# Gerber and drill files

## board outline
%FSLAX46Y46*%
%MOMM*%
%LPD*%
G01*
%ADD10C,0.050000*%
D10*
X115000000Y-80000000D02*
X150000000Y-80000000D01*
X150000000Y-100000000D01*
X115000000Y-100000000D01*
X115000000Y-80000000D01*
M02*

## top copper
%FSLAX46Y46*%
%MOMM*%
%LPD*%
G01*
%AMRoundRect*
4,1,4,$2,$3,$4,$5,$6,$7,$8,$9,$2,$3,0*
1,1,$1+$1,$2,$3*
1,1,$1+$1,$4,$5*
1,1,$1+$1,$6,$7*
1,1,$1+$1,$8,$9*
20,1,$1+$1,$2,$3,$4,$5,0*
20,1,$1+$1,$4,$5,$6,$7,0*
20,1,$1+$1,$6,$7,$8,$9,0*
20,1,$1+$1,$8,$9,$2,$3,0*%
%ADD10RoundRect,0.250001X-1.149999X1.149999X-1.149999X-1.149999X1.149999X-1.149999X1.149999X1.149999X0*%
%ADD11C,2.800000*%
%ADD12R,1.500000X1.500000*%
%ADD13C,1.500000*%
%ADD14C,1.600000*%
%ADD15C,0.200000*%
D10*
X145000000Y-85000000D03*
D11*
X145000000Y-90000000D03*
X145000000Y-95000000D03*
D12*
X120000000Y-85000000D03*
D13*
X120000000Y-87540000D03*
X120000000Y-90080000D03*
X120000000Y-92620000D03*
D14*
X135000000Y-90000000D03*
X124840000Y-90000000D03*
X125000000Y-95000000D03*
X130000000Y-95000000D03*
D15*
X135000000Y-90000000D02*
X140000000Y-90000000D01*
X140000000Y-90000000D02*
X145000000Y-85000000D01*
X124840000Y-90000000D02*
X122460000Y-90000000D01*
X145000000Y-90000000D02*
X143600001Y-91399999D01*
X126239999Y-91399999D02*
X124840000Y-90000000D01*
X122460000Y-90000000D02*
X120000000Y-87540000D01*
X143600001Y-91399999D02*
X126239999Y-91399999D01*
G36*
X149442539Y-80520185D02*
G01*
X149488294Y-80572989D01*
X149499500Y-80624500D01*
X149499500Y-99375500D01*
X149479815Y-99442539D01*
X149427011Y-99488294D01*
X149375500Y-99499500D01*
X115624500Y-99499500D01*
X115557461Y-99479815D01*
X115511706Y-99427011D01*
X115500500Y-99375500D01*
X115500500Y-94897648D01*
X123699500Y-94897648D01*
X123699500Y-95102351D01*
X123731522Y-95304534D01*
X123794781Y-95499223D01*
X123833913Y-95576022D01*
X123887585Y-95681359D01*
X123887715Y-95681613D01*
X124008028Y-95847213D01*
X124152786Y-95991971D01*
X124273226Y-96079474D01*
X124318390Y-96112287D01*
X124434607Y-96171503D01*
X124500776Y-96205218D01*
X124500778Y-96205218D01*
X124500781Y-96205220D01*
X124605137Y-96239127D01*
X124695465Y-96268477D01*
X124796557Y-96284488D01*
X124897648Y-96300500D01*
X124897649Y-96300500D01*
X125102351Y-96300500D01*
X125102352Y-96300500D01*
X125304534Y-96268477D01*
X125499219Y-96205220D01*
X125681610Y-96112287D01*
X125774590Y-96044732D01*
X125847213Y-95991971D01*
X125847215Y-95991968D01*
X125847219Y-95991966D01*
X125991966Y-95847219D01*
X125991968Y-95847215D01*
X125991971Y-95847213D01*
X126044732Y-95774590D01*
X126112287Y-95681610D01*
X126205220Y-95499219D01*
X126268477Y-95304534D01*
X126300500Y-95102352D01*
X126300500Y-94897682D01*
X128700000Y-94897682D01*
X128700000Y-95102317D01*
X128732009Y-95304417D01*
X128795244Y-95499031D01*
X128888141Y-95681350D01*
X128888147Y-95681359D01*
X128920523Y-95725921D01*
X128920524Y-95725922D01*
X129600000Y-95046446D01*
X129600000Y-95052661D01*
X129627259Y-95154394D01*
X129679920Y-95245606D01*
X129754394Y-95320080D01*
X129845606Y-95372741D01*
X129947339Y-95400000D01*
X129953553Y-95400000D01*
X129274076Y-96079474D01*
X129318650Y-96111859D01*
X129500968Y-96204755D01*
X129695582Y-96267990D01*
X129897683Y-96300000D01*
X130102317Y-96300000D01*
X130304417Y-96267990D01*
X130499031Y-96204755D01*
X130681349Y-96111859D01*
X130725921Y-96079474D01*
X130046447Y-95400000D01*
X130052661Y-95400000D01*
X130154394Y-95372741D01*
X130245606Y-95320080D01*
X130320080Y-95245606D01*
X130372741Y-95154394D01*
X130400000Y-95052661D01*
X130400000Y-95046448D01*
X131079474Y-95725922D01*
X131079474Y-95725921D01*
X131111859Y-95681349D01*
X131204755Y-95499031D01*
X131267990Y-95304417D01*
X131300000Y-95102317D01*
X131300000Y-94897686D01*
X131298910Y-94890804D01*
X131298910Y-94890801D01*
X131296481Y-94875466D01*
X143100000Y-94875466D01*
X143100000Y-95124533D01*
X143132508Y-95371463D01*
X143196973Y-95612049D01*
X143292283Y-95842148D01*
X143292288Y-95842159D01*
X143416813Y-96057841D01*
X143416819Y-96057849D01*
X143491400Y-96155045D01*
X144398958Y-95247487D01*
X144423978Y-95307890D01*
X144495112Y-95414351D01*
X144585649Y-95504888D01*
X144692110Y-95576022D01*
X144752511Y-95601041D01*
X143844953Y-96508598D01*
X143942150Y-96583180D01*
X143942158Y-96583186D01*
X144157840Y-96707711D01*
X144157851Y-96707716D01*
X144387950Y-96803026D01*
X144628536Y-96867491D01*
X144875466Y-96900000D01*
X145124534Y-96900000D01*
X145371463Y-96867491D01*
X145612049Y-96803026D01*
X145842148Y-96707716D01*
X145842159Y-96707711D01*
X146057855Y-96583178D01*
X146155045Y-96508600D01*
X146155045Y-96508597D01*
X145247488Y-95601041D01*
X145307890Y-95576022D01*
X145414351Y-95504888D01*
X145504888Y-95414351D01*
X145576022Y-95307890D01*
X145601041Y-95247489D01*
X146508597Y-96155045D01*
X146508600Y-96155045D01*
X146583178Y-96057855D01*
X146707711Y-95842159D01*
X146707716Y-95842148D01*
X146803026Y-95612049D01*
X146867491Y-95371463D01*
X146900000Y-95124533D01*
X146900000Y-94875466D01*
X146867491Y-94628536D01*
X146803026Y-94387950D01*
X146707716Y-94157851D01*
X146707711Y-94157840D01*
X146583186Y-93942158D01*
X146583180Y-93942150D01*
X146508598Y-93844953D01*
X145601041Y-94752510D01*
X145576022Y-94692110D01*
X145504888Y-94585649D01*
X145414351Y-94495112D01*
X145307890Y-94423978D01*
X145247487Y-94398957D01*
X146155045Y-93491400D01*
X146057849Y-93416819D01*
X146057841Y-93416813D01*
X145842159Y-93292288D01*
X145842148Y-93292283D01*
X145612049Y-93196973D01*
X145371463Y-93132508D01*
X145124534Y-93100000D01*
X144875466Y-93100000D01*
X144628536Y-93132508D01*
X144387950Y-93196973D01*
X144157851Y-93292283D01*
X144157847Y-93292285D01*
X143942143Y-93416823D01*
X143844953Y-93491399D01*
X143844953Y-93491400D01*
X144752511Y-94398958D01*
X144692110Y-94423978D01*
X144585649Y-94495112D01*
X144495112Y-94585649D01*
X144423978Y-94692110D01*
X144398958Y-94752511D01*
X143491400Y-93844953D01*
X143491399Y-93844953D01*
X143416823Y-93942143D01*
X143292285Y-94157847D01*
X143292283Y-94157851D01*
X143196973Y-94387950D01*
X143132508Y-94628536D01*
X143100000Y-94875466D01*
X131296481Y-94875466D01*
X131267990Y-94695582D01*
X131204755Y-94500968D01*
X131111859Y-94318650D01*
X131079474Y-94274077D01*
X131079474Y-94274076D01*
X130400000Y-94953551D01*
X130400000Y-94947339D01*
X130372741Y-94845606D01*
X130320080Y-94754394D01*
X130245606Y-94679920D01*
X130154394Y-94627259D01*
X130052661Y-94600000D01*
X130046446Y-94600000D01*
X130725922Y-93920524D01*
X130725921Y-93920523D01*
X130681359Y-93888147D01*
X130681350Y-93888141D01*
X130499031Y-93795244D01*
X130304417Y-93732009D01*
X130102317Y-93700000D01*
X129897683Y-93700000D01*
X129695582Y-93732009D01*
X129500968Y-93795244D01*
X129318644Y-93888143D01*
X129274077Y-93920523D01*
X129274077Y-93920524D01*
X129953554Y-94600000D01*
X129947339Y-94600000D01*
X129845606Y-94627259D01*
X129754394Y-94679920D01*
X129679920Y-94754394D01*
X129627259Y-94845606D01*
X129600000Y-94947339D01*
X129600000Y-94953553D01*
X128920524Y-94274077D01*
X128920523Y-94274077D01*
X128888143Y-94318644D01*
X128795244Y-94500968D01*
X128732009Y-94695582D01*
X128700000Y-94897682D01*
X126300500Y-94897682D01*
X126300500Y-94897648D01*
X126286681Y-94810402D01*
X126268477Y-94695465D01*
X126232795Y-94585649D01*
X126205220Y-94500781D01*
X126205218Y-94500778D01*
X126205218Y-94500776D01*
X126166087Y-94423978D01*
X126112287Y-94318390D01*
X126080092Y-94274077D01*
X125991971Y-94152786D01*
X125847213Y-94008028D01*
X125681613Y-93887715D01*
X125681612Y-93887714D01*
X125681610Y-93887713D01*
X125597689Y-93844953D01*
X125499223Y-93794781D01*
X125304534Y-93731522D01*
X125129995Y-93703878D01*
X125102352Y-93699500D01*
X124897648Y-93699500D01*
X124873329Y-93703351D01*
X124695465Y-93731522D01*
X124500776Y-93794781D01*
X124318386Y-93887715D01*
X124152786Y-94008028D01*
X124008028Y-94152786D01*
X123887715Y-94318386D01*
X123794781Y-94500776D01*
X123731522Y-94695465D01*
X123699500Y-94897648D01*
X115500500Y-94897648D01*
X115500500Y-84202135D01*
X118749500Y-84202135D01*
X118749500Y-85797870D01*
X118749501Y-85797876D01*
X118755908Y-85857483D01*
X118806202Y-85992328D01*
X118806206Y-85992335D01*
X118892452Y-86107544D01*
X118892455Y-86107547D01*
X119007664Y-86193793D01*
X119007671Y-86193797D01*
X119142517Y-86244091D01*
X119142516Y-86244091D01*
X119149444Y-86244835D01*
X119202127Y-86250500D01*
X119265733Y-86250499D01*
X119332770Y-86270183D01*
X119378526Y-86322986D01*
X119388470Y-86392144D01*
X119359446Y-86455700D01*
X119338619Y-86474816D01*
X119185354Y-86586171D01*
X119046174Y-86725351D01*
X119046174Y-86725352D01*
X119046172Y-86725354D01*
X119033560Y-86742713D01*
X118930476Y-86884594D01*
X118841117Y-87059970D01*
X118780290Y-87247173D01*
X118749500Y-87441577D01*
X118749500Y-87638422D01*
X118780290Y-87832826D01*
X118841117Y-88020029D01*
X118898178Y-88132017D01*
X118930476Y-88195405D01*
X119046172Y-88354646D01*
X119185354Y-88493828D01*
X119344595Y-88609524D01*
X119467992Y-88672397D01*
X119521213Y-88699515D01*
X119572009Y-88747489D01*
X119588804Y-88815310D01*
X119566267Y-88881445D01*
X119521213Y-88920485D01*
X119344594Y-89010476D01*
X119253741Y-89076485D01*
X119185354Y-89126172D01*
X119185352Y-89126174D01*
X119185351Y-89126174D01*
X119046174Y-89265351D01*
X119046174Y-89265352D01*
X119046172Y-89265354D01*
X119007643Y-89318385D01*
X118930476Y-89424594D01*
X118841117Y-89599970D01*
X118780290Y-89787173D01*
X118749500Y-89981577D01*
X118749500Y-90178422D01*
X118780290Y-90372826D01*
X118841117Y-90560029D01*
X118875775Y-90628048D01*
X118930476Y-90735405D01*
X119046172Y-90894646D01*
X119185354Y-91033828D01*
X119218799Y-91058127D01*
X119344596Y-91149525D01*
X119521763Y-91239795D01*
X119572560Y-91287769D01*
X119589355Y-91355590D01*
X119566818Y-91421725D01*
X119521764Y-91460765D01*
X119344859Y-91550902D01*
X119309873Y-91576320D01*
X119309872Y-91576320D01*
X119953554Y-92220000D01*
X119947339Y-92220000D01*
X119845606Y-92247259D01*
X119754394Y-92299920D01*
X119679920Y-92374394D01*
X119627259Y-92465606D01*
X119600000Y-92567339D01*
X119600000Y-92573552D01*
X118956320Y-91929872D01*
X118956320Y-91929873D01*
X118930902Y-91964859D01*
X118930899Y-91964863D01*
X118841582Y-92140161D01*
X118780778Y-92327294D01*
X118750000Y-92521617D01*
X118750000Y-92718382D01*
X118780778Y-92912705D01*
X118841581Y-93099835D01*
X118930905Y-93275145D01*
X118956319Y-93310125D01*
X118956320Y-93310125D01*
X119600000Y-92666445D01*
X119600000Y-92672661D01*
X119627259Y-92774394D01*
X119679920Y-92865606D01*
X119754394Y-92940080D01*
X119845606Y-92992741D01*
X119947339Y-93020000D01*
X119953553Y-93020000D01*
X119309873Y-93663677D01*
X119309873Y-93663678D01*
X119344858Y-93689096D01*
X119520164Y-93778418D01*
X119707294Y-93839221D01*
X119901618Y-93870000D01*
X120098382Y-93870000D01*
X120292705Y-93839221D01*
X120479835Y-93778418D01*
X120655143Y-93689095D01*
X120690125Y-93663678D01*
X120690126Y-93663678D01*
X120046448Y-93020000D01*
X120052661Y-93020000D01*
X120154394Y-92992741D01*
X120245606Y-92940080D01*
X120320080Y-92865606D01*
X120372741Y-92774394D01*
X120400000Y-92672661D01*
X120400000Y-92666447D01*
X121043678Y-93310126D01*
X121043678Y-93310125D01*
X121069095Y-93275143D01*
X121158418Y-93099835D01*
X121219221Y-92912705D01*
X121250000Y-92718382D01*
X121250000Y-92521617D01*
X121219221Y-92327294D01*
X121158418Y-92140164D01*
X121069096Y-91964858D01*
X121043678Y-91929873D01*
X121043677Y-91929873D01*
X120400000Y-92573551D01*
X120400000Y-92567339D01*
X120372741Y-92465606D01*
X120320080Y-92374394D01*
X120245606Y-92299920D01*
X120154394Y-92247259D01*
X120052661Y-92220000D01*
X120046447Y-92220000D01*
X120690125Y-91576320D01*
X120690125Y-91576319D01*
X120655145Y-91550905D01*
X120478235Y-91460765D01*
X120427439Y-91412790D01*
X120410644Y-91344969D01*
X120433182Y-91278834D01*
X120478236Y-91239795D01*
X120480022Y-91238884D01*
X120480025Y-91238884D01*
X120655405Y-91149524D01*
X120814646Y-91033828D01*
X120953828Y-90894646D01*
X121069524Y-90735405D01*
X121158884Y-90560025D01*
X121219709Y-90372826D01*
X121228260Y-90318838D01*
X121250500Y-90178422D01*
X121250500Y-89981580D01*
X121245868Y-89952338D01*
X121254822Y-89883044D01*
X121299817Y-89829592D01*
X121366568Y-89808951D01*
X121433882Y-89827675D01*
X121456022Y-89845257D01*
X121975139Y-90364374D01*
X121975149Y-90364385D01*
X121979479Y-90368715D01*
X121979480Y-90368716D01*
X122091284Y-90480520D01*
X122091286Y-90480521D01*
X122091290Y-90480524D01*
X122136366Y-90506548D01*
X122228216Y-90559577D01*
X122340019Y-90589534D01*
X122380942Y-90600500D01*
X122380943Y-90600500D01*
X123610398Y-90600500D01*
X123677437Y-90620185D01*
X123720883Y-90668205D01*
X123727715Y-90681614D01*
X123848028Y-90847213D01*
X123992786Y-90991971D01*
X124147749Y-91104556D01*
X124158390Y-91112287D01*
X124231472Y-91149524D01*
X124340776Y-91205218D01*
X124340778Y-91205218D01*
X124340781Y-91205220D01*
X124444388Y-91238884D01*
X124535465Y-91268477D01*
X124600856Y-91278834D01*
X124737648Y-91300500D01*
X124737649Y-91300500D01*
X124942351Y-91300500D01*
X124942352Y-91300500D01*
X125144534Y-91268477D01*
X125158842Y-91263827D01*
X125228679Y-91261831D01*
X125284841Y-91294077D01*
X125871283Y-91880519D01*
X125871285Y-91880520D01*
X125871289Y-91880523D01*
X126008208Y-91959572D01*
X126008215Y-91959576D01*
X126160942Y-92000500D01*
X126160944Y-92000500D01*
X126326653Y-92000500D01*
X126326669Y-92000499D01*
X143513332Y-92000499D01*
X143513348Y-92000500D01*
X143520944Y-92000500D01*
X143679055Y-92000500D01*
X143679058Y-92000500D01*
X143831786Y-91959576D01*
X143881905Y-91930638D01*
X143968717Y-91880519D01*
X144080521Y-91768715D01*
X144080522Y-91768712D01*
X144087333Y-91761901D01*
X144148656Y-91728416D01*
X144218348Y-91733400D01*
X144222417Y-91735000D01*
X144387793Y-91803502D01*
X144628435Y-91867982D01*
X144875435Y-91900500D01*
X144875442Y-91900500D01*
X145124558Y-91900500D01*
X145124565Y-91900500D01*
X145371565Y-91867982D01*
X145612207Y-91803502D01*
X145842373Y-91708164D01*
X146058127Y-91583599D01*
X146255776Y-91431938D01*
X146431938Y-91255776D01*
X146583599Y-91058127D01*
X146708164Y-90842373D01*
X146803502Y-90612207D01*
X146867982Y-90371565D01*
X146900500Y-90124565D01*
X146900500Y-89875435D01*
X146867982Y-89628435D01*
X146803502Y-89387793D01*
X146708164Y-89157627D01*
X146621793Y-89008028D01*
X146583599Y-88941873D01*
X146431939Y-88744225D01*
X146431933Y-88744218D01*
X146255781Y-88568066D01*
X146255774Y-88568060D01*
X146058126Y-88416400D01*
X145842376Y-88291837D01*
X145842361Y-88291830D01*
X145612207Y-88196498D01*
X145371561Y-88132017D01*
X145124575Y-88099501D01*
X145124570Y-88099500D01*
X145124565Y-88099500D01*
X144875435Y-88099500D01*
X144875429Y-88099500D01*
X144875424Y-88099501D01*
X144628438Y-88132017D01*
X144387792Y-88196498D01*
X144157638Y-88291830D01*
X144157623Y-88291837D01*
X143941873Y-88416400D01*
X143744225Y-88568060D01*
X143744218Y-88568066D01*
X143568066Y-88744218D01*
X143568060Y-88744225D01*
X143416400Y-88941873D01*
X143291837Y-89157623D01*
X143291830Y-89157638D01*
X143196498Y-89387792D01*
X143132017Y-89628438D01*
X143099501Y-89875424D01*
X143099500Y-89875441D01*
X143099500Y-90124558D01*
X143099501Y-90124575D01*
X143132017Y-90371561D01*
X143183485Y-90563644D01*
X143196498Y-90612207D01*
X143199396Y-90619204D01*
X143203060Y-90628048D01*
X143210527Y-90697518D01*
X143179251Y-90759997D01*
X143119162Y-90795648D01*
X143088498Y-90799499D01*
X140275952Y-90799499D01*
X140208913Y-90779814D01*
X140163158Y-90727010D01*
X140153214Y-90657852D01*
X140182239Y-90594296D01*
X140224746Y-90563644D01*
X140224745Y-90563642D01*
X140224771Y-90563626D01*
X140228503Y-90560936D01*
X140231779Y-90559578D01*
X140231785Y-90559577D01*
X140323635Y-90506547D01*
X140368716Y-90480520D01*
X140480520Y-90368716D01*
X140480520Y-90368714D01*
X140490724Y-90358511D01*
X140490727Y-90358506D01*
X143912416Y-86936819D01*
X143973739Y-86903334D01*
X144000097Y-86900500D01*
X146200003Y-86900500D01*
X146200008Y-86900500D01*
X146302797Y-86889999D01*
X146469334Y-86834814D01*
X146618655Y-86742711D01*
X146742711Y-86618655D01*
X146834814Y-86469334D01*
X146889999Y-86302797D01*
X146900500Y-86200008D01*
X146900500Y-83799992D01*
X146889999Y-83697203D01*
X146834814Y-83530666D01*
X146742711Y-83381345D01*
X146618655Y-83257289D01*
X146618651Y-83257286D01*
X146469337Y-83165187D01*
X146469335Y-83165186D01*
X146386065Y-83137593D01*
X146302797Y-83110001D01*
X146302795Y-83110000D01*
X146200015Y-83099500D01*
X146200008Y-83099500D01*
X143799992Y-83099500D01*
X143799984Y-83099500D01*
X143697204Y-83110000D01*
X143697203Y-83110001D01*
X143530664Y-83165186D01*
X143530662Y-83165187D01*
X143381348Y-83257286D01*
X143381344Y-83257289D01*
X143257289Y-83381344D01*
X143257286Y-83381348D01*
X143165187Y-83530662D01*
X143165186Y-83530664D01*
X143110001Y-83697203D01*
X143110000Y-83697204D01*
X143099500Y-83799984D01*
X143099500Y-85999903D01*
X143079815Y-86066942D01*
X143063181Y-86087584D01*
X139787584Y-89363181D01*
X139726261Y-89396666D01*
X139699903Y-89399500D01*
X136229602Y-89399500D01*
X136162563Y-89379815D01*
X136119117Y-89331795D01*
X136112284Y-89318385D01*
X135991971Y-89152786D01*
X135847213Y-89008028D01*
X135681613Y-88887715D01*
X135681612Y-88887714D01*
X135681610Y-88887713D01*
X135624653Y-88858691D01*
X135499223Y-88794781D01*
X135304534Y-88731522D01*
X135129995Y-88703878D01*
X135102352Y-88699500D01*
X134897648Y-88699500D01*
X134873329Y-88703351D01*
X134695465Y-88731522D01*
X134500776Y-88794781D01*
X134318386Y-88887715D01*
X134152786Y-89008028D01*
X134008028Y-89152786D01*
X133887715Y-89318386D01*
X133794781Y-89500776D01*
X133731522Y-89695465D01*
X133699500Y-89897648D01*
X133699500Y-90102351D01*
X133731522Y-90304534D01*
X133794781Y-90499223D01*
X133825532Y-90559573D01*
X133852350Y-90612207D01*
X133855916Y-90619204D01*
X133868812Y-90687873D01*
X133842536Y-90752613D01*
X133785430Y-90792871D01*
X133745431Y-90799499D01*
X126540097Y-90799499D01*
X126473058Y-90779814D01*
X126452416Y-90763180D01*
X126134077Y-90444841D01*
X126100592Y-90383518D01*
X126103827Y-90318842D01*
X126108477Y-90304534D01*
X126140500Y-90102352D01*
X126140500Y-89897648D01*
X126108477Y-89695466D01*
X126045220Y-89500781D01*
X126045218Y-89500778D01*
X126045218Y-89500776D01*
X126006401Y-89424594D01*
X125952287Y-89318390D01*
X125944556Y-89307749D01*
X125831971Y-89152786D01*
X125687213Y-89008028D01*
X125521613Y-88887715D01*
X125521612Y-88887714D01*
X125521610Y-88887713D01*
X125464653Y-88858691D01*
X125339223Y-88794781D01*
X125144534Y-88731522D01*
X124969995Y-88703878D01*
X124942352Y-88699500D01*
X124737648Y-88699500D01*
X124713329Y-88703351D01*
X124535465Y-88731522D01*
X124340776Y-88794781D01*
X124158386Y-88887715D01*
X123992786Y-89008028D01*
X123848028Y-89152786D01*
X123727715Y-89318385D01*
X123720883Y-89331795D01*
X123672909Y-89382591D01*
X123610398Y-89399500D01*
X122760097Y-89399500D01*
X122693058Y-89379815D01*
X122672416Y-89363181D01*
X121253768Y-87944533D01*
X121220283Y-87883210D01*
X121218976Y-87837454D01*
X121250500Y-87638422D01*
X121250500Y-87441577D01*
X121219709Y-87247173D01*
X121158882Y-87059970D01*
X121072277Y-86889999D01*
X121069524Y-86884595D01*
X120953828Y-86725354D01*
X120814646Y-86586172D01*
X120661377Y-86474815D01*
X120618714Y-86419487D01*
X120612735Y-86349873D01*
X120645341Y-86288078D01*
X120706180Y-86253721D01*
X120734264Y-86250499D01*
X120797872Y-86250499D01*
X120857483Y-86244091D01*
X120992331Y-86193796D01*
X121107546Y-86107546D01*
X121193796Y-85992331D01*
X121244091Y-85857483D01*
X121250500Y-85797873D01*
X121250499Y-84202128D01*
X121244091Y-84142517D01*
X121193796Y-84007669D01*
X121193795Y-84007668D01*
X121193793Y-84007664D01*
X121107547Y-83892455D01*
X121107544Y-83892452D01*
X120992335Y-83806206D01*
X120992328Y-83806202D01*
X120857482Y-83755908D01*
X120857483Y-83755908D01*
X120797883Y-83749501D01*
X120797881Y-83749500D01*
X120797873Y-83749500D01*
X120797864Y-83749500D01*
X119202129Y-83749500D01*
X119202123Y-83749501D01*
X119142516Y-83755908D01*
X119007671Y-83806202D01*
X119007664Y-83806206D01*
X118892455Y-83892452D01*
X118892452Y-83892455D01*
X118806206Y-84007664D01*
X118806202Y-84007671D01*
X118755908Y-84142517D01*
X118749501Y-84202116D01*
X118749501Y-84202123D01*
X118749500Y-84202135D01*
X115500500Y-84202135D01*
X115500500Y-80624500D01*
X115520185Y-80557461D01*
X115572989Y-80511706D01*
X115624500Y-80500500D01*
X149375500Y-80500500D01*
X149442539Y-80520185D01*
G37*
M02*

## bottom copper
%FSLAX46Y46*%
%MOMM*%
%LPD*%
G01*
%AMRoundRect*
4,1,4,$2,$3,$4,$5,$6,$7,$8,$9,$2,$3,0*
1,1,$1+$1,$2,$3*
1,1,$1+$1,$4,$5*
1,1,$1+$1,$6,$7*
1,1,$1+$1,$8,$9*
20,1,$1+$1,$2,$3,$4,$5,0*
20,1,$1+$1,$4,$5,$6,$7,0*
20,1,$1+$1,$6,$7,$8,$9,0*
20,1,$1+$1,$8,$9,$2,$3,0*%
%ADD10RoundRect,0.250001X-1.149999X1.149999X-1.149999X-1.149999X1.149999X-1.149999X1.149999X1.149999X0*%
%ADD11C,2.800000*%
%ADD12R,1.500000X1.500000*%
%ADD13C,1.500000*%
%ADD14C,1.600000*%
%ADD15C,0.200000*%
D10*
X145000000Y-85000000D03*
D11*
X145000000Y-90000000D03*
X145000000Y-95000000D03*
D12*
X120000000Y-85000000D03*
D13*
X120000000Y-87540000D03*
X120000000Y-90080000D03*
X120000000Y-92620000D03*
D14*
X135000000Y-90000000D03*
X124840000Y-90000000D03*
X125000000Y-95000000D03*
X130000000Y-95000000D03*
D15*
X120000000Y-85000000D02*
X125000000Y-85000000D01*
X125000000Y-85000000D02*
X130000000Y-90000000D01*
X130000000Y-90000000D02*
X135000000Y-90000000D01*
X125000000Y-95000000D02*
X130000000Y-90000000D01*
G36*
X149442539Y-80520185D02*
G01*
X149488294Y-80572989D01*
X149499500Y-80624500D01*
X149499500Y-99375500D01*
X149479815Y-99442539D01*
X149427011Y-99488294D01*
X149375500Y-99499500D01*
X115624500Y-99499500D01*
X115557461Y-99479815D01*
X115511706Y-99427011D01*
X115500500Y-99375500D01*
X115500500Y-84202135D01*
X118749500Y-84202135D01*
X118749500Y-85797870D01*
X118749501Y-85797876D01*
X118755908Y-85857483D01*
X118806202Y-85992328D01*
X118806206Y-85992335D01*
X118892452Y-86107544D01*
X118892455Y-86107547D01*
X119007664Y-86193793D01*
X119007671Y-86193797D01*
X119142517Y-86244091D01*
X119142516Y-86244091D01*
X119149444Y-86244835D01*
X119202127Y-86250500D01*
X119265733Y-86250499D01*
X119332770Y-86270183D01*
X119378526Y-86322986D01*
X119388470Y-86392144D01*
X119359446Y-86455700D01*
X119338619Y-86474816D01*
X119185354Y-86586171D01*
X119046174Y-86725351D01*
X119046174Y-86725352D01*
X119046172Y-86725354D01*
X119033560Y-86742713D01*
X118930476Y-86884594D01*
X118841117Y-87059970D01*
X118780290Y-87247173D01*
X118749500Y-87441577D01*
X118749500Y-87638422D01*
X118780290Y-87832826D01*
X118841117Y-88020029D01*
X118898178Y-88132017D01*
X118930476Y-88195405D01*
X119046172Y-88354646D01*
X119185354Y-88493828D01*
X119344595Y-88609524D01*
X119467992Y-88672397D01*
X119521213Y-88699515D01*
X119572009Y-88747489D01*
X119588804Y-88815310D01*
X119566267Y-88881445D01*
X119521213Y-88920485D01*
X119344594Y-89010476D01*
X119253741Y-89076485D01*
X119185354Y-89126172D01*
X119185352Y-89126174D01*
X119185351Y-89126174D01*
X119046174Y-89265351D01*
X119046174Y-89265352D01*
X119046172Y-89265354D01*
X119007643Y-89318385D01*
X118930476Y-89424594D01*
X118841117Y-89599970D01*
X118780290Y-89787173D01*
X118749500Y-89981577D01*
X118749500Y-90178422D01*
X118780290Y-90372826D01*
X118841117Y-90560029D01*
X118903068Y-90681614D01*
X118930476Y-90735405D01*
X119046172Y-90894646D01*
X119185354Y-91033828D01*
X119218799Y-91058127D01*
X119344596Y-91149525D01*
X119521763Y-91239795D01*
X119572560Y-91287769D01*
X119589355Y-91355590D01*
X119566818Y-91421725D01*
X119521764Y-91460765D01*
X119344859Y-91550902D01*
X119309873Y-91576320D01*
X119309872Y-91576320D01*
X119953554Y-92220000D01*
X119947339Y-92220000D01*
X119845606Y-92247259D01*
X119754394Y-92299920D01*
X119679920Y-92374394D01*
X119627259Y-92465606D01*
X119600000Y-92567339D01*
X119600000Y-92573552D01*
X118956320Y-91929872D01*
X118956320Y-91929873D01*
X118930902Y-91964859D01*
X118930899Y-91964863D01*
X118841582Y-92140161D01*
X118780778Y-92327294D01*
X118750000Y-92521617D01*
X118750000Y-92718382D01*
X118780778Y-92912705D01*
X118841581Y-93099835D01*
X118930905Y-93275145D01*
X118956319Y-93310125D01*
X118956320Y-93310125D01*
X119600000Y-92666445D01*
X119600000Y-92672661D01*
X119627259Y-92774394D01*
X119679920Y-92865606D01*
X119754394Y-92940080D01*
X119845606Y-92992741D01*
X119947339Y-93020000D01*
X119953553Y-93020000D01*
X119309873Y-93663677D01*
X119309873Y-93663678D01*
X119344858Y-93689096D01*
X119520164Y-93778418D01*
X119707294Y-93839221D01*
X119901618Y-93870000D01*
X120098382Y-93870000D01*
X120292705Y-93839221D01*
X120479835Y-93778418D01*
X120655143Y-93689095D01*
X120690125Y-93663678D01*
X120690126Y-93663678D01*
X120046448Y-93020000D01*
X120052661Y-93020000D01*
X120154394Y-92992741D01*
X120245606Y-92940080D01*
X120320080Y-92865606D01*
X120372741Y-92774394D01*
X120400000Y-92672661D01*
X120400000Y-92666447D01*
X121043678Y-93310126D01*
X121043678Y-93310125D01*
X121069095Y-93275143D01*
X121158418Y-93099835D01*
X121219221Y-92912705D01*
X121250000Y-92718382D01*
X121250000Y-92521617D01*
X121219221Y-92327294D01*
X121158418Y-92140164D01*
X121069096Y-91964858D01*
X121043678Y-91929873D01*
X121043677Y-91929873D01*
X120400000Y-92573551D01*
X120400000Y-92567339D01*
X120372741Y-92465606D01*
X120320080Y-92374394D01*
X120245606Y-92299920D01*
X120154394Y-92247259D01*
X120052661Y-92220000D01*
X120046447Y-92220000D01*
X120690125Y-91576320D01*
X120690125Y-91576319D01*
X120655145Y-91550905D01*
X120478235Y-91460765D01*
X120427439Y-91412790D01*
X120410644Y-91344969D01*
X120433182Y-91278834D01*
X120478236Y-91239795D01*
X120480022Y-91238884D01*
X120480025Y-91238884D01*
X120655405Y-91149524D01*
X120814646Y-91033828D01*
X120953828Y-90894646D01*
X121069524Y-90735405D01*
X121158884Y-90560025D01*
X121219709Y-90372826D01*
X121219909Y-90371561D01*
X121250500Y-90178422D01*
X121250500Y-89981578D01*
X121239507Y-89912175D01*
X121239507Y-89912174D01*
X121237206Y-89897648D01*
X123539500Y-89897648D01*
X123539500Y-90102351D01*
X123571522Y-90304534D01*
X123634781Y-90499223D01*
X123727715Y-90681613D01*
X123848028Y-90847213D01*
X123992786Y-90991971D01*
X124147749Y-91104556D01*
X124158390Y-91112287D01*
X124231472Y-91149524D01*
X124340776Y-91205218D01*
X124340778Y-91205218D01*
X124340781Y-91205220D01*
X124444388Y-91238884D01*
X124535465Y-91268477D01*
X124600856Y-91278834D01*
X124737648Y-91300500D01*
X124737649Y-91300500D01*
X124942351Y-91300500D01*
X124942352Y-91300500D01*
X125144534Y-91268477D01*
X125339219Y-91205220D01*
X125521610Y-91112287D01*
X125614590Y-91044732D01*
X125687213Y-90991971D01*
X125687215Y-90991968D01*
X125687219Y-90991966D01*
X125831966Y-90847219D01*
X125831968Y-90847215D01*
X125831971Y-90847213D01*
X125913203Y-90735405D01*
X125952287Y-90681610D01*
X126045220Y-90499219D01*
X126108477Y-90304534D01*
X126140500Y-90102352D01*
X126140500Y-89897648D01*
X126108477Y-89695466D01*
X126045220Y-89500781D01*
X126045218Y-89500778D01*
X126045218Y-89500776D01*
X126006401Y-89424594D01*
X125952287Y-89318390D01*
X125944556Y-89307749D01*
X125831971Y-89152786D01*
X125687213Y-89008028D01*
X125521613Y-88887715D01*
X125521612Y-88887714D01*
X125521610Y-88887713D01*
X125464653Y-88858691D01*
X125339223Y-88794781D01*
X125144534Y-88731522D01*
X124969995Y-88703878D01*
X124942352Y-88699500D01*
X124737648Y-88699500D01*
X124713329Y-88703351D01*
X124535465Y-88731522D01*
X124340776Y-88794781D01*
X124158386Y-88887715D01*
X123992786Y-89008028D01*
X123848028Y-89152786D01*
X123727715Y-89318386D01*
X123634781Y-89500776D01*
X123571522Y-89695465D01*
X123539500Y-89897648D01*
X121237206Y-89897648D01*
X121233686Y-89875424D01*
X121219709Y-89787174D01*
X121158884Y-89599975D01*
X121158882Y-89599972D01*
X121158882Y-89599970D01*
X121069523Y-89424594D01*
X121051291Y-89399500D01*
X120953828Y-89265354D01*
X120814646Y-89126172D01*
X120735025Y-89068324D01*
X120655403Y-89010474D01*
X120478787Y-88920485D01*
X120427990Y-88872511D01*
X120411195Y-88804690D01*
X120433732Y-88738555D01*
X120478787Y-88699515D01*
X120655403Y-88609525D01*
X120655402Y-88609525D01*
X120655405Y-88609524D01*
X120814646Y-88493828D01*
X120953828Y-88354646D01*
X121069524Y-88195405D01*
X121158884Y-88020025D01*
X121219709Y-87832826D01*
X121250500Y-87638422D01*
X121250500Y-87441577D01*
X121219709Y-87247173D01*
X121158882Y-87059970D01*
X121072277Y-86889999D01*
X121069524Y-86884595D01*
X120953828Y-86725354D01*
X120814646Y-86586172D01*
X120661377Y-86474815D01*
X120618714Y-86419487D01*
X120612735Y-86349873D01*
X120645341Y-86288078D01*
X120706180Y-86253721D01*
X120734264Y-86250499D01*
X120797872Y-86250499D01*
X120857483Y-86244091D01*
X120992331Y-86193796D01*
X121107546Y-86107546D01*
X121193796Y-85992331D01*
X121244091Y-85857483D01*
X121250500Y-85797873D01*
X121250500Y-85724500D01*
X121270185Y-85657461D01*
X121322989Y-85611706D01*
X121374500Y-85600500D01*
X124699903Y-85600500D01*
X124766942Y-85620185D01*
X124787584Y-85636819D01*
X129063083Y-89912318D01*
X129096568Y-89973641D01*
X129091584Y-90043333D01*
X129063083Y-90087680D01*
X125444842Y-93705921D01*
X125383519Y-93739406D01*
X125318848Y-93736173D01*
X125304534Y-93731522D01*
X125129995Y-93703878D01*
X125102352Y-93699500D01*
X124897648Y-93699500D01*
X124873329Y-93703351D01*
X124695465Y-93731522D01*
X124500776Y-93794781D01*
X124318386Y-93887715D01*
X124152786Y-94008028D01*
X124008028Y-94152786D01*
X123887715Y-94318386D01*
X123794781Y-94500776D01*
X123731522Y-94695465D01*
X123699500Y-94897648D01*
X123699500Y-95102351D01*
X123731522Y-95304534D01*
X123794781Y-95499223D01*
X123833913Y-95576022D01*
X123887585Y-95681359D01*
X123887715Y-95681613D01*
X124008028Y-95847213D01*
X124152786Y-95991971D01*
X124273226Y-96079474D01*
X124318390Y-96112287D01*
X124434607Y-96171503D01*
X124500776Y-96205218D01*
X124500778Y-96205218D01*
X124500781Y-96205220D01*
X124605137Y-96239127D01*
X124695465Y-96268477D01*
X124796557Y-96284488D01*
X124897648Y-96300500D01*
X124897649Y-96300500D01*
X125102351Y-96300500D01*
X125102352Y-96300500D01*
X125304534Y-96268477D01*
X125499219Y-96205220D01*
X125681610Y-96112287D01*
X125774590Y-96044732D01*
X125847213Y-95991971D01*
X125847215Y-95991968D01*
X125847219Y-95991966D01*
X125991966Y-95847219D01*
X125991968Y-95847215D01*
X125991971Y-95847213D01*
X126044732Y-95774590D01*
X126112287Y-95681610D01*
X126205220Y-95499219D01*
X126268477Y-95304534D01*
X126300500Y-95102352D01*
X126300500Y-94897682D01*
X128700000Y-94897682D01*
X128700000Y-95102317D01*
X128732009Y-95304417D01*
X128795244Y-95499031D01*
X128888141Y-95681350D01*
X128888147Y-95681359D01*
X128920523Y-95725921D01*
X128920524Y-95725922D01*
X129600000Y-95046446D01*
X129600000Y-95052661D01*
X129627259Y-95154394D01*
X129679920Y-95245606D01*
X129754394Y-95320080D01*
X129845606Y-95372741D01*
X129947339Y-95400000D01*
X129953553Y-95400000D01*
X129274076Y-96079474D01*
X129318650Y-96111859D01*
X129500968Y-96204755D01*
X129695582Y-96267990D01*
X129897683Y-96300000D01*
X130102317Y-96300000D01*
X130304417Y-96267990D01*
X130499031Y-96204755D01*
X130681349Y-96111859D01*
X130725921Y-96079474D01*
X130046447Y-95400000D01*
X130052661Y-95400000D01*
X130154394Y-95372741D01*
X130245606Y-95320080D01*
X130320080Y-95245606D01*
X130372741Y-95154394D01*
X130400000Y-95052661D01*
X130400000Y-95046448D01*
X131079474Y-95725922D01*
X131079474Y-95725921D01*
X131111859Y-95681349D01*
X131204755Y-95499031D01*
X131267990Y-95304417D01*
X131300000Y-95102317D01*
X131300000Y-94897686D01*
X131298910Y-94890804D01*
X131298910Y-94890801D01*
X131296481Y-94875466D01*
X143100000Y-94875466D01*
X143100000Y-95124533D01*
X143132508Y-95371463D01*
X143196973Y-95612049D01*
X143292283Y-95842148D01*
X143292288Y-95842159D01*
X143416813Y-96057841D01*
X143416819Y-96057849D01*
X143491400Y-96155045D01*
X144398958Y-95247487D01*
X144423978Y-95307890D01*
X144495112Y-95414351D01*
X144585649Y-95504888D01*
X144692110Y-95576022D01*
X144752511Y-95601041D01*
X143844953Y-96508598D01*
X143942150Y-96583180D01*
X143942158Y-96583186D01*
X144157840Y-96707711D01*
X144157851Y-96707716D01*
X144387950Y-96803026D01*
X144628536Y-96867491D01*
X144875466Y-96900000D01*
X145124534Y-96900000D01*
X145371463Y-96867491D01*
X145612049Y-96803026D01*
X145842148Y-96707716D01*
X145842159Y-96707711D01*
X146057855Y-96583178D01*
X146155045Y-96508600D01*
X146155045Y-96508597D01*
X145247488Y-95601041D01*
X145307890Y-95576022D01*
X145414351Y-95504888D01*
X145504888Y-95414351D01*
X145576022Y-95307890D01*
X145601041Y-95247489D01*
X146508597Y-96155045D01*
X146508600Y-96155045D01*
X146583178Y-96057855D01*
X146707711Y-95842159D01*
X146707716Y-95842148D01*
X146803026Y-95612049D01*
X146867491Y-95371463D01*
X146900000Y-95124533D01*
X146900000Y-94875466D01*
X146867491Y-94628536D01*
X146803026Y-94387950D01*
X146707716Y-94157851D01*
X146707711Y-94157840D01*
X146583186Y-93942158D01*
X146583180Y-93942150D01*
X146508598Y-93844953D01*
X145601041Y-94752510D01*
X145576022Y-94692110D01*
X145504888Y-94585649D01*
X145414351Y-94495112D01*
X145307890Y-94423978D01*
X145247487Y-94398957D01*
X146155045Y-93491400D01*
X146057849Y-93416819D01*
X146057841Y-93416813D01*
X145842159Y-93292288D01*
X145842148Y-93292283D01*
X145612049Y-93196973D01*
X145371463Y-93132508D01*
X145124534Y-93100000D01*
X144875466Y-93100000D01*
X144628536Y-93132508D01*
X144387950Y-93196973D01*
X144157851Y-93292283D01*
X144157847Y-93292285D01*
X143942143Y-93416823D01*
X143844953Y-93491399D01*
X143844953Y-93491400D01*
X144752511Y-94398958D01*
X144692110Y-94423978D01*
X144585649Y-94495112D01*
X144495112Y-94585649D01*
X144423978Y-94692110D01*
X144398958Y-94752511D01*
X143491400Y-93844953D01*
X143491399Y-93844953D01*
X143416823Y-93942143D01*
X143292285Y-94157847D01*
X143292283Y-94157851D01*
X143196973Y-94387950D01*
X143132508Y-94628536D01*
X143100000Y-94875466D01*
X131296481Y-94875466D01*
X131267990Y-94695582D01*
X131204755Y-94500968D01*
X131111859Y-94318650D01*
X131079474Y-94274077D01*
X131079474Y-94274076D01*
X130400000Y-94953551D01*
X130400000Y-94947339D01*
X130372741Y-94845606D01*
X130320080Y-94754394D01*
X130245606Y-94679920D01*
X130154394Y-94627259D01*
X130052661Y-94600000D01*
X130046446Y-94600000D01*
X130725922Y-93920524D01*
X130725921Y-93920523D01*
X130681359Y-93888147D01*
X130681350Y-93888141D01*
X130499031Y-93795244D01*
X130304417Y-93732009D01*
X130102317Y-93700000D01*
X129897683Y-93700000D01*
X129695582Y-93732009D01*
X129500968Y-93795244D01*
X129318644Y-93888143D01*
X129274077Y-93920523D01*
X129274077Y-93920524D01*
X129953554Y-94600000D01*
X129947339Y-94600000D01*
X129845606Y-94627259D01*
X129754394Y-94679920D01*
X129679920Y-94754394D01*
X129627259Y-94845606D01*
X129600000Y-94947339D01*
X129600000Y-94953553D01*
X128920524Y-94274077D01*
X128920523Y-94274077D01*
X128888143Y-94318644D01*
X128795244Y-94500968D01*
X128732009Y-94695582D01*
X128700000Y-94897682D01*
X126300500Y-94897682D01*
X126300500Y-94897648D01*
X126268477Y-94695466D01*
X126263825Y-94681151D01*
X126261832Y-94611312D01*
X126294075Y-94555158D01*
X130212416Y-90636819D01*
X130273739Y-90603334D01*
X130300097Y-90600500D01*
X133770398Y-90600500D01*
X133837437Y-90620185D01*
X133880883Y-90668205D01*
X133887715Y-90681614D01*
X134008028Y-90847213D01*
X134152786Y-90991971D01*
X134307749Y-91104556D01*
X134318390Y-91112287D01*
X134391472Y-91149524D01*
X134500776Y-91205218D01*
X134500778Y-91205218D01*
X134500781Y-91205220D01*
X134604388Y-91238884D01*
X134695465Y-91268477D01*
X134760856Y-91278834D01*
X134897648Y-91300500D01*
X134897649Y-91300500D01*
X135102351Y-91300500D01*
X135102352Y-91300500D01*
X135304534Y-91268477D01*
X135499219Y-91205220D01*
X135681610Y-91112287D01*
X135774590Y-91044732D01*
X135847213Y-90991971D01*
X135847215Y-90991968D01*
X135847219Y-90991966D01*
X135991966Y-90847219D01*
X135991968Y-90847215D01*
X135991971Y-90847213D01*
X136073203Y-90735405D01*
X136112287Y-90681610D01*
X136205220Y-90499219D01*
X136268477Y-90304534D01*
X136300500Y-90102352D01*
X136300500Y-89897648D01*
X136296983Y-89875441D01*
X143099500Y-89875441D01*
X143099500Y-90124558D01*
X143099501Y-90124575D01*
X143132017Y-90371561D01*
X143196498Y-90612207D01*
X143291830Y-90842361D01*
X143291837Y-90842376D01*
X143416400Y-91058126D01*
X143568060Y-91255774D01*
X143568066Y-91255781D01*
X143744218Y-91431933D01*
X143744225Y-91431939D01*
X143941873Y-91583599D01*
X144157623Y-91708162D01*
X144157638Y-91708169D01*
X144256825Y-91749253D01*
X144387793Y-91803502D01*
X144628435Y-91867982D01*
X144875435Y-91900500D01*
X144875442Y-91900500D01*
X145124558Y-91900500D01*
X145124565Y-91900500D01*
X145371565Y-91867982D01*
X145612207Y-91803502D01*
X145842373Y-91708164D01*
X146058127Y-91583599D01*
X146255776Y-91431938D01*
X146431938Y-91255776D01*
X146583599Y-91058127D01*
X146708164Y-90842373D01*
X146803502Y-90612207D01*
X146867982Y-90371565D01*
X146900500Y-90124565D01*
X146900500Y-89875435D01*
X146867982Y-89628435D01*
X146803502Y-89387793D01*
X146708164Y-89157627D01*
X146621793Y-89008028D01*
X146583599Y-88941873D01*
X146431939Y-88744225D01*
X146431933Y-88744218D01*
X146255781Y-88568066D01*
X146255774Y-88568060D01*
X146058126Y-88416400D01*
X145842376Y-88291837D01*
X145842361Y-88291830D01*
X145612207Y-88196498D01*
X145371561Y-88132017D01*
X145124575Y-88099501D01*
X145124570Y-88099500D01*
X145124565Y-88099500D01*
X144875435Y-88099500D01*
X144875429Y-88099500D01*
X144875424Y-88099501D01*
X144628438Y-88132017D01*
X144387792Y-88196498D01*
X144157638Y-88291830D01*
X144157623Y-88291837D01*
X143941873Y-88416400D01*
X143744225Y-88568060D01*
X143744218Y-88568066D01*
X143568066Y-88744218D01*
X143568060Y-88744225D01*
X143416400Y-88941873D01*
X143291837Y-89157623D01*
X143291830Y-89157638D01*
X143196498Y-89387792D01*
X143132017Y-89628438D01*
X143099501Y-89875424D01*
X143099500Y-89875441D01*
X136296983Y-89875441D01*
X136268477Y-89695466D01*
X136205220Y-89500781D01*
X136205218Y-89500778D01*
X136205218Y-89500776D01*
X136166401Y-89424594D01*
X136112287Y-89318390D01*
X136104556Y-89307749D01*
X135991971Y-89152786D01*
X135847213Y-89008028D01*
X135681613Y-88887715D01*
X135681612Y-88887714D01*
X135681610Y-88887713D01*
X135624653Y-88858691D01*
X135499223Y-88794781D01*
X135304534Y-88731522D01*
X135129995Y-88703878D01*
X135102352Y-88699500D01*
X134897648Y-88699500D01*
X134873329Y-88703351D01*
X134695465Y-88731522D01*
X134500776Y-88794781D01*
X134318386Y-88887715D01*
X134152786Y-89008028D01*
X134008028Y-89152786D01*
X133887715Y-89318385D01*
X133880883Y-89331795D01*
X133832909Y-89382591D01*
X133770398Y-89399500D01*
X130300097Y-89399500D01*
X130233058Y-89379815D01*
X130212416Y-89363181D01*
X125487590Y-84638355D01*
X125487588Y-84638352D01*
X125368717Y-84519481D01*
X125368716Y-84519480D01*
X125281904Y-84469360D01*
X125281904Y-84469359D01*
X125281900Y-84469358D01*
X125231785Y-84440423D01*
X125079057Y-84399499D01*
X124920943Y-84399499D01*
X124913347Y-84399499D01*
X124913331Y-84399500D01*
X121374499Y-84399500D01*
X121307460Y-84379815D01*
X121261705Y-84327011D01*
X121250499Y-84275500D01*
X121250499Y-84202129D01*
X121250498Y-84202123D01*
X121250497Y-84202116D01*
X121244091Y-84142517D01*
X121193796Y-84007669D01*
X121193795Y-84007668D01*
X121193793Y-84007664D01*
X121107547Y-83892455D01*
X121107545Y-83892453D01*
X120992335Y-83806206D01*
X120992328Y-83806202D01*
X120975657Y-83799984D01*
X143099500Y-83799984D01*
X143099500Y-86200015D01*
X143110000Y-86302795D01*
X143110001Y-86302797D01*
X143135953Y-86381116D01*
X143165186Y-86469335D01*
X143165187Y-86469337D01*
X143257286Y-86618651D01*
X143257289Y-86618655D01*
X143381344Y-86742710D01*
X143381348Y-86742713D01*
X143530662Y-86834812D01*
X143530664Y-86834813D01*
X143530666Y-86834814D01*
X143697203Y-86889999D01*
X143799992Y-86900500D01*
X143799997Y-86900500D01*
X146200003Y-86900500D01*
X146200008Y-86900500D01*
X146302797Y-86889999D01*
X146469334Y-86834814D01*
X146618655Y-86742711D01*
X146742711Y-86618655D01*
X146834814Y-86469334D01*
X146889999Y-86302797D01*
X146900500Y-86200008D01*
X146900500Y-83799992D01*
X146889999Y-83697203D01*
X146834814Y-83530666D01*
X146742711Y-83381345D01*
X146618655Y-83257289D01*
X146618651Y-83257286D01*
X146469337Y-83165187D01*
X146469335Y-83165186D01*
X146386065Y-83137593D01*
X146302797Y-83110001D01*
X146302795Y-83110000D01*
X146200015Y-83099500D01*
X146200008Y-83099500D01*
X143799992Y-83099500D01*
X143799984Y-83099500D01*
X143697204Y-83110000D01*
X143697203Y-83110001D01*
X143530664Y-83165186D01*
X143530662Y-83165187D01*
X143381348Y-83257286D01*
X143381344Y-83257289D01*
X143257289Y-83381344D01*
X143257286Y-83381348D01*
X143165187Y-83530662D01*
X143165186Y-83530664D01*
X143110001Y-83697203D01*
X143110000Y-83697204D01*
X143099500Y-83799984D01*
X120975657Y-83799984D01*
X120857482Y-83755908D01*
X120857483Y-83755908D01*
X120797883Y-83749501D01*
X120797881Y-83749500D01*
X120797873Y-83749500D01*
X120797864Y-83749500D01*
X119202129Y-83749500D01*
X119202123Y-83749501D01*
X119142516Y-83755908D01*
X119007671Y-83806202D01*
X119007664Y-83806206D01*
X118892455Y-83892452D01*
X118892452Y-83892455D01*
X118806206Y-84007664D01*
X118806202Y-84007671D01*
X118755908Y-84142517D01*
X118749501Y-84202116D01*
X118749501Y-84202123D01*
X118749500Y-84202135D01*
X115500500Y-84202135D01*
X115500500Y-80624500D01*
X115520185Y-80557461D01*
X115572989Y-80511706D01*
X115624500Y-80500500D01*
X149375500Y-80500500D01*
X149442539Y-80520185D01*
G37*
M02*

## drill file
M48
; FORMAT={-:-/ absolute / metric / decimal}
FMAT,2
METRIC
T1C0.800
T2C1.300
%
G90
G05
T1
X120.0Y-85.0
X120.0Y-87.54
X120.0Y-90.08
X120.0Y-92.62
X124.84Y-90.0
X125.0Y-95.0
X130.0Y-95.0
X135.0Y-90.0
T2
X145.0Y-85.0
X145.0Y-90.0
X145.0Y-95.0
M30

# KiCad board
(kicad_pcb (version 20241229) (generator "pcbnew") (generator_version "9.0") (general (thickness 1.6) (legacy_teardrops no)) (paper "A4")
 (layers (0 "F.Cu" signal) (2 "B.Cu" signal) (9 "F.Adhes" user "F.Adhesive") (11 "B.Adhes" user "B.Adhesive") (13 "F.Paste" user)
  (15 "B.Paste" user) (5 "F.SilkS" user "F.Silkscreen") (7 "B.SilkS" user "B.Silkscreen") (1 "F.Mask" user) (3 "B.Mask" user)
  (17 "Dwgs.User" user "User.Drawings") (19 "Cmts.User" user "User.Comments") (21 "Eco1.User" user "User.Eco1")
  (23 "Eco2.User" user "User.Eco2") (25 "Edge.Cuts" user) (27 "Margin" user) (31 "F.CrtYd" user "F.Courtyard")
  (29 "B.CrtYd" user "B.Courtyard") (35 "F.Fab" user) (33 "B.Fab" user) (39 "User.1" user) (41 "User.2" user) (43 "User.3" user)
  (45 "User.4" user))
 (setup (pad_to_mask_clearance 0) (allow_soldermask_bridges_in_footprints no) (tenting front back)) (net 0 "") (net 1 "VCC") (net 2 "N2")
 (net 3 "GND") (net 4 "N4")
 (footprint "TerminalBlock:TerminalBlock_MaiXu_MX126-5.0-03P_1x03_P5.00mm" (layer "F.Cu") (at 145 85 -90)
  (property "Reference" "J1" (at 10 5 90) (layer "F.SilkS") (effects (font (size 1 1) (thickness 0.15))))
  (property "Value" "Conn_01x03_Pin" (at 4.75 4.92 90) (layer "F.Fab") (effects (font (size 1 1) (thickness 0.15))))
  (pad "1" thru_hole roundrect (at 0 0 270) (size 2.8 2.8) (drill 1.3) (layers "*.Cu" "*.Mask") (remove_unused_layers no)
   (roundrect_rratio 0.089286) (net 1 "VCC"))
  (pad "2" thru_hole circle (at 5 0 270) (size 2.8 2.8) (drill 1.3) (layers "*.Cu" "*.Mask") (remove_unused_layers no) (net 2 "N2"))
  (pad "3" thru_hole circle (at 10 0 270) (size 2.8 2.8) (drill 1.3) (layers "*.Cu" "*.Mask") (remove_unused_layers no) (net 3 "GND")))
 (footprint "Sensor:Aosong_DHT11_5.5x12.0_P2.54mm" (layer "F.Cu") (at 120 85)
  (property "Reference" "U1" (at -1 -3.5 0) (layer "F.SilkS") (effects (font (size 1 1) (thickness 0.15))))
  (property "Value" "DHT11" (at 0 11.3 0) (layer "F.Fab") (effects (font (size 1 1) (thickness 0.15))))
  (pad "1" thru_hole rect (at 0 0) (size 1.5 1.5) (drill 0.8) (layers "*.Cu" "*.Mask") (remove_unused_layers no) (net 1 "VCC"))
  (pad "2" thru_hole circle (at 0 2.54) (size 1.5 1.5) (drill 0.8) (layers "*.Cu" "*.Mask") (remove_unused_layers no) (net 2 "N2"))
  (pad "3" thru_hole circle (at 0 5.08) (size 1.5 1.5) (drill 0.8) (layers "*.Cu" "*.Mask") (remove_unused_layers no) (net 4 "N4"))
  (pad "4" thru_hole circle (at 0 7.62) (size 1.5 1.5) (drill 0.8) (layers "*.Cu" "*.Mask") (remove_unused_layers no) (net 3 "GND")))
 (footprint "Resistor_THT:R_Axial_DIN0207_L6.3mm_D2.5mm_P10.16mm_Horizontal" (layer "F.Cu") (at 135 90 180)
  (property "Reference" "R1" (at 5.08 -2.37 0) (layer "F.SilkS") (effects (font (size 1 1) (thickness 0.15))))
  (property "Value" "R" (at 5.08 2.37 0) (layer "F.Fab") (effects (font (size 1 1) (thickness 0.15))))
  (pad "1" thru_hole circle (at 0 0 180) (size 1.6 1.6) (drill 0.8) (layers "*.Cu" "*.Mask") (remove_unused_layers no) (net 1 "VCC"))
  (pad "2" thru_hole circle (at 10.16 0 180) (size 1.6 1.6) (drill 0.8) (layers "*.Cu" "*.Mask") (remove_unused_layers no) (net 2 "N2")))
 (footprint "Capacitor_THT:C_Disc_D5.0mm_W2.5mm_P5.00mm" (layer "F.Cu") (at 125 95)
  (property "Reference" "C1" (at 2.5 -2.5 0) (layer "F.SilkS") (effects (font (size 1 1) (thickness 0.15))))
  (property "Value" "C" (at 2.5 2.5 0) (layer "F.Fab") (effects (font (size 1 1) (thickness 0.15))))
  (pad "1" thru_hole circle (at 0 0) (size 1.6 1.6) (drill 0.8) (layers "*.Cu" "*.Mask") (remove_unused_layers no) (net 1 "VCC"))
  (pad "2" thru_hole circle (at 5 0) (size 1.6 1.6) (drill 0.8) (layers "*.Cu" "*.Mask") (remove_unused_layers no) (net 3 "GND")))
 (gr_rect (start 115 80) (end 150 100) (stroke (width 0.05) (type default)) (fill no) (layer "Edge.Cuts"))
 (segment (start 135 90) (end 140 90) (width 0.2) (layer "F.Cu") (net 1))
 (segment (start 140 90) (end 145 85) (width 0.2) (layer "F.Cu") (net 1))
 (segment (start 120 85) (end 125 85) (width 0.2) (layer "B.Cu") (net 1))
 (segment (start 125 85) (end 130 90) (width 0.2) (layer "B.Cu") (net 1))
 (segment (start 130 90) (end 135 90) (width 0.2) (layer "B.Cu") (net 1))
 (segment (start 125 95) (end 130 90) (width 0.2) (layer "B.Cu") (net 1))
 (segment (start 124.84 90) (end 122.46 90) (width 0.2) (layer "F.Cu") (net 2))
 (segment (start 145 90) (end 143.600001 91.399999) (width 0.2) (layer "F.Cu") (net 2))
 (segment (start 126.239999 91.399999) (end 124.84 90) (width 0.2) (layer "F.Cu") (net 2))
 (segment (start 122.46 90) (end 120 87.54) (width 0.2) (layer "F.Cu") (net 2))
 (segment (start 143.600001 91.399999) (end 126.239999 91.399999) (width 0.2) (layer "F.Cu") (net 2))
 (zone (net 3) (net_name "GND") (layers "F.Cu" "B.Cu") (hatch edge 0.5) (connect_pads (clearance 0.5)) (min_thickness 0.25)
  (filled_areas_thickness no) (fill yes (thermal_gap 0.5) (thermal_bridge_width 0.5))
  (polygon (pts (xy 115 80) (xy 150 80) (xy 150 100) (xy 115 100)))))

